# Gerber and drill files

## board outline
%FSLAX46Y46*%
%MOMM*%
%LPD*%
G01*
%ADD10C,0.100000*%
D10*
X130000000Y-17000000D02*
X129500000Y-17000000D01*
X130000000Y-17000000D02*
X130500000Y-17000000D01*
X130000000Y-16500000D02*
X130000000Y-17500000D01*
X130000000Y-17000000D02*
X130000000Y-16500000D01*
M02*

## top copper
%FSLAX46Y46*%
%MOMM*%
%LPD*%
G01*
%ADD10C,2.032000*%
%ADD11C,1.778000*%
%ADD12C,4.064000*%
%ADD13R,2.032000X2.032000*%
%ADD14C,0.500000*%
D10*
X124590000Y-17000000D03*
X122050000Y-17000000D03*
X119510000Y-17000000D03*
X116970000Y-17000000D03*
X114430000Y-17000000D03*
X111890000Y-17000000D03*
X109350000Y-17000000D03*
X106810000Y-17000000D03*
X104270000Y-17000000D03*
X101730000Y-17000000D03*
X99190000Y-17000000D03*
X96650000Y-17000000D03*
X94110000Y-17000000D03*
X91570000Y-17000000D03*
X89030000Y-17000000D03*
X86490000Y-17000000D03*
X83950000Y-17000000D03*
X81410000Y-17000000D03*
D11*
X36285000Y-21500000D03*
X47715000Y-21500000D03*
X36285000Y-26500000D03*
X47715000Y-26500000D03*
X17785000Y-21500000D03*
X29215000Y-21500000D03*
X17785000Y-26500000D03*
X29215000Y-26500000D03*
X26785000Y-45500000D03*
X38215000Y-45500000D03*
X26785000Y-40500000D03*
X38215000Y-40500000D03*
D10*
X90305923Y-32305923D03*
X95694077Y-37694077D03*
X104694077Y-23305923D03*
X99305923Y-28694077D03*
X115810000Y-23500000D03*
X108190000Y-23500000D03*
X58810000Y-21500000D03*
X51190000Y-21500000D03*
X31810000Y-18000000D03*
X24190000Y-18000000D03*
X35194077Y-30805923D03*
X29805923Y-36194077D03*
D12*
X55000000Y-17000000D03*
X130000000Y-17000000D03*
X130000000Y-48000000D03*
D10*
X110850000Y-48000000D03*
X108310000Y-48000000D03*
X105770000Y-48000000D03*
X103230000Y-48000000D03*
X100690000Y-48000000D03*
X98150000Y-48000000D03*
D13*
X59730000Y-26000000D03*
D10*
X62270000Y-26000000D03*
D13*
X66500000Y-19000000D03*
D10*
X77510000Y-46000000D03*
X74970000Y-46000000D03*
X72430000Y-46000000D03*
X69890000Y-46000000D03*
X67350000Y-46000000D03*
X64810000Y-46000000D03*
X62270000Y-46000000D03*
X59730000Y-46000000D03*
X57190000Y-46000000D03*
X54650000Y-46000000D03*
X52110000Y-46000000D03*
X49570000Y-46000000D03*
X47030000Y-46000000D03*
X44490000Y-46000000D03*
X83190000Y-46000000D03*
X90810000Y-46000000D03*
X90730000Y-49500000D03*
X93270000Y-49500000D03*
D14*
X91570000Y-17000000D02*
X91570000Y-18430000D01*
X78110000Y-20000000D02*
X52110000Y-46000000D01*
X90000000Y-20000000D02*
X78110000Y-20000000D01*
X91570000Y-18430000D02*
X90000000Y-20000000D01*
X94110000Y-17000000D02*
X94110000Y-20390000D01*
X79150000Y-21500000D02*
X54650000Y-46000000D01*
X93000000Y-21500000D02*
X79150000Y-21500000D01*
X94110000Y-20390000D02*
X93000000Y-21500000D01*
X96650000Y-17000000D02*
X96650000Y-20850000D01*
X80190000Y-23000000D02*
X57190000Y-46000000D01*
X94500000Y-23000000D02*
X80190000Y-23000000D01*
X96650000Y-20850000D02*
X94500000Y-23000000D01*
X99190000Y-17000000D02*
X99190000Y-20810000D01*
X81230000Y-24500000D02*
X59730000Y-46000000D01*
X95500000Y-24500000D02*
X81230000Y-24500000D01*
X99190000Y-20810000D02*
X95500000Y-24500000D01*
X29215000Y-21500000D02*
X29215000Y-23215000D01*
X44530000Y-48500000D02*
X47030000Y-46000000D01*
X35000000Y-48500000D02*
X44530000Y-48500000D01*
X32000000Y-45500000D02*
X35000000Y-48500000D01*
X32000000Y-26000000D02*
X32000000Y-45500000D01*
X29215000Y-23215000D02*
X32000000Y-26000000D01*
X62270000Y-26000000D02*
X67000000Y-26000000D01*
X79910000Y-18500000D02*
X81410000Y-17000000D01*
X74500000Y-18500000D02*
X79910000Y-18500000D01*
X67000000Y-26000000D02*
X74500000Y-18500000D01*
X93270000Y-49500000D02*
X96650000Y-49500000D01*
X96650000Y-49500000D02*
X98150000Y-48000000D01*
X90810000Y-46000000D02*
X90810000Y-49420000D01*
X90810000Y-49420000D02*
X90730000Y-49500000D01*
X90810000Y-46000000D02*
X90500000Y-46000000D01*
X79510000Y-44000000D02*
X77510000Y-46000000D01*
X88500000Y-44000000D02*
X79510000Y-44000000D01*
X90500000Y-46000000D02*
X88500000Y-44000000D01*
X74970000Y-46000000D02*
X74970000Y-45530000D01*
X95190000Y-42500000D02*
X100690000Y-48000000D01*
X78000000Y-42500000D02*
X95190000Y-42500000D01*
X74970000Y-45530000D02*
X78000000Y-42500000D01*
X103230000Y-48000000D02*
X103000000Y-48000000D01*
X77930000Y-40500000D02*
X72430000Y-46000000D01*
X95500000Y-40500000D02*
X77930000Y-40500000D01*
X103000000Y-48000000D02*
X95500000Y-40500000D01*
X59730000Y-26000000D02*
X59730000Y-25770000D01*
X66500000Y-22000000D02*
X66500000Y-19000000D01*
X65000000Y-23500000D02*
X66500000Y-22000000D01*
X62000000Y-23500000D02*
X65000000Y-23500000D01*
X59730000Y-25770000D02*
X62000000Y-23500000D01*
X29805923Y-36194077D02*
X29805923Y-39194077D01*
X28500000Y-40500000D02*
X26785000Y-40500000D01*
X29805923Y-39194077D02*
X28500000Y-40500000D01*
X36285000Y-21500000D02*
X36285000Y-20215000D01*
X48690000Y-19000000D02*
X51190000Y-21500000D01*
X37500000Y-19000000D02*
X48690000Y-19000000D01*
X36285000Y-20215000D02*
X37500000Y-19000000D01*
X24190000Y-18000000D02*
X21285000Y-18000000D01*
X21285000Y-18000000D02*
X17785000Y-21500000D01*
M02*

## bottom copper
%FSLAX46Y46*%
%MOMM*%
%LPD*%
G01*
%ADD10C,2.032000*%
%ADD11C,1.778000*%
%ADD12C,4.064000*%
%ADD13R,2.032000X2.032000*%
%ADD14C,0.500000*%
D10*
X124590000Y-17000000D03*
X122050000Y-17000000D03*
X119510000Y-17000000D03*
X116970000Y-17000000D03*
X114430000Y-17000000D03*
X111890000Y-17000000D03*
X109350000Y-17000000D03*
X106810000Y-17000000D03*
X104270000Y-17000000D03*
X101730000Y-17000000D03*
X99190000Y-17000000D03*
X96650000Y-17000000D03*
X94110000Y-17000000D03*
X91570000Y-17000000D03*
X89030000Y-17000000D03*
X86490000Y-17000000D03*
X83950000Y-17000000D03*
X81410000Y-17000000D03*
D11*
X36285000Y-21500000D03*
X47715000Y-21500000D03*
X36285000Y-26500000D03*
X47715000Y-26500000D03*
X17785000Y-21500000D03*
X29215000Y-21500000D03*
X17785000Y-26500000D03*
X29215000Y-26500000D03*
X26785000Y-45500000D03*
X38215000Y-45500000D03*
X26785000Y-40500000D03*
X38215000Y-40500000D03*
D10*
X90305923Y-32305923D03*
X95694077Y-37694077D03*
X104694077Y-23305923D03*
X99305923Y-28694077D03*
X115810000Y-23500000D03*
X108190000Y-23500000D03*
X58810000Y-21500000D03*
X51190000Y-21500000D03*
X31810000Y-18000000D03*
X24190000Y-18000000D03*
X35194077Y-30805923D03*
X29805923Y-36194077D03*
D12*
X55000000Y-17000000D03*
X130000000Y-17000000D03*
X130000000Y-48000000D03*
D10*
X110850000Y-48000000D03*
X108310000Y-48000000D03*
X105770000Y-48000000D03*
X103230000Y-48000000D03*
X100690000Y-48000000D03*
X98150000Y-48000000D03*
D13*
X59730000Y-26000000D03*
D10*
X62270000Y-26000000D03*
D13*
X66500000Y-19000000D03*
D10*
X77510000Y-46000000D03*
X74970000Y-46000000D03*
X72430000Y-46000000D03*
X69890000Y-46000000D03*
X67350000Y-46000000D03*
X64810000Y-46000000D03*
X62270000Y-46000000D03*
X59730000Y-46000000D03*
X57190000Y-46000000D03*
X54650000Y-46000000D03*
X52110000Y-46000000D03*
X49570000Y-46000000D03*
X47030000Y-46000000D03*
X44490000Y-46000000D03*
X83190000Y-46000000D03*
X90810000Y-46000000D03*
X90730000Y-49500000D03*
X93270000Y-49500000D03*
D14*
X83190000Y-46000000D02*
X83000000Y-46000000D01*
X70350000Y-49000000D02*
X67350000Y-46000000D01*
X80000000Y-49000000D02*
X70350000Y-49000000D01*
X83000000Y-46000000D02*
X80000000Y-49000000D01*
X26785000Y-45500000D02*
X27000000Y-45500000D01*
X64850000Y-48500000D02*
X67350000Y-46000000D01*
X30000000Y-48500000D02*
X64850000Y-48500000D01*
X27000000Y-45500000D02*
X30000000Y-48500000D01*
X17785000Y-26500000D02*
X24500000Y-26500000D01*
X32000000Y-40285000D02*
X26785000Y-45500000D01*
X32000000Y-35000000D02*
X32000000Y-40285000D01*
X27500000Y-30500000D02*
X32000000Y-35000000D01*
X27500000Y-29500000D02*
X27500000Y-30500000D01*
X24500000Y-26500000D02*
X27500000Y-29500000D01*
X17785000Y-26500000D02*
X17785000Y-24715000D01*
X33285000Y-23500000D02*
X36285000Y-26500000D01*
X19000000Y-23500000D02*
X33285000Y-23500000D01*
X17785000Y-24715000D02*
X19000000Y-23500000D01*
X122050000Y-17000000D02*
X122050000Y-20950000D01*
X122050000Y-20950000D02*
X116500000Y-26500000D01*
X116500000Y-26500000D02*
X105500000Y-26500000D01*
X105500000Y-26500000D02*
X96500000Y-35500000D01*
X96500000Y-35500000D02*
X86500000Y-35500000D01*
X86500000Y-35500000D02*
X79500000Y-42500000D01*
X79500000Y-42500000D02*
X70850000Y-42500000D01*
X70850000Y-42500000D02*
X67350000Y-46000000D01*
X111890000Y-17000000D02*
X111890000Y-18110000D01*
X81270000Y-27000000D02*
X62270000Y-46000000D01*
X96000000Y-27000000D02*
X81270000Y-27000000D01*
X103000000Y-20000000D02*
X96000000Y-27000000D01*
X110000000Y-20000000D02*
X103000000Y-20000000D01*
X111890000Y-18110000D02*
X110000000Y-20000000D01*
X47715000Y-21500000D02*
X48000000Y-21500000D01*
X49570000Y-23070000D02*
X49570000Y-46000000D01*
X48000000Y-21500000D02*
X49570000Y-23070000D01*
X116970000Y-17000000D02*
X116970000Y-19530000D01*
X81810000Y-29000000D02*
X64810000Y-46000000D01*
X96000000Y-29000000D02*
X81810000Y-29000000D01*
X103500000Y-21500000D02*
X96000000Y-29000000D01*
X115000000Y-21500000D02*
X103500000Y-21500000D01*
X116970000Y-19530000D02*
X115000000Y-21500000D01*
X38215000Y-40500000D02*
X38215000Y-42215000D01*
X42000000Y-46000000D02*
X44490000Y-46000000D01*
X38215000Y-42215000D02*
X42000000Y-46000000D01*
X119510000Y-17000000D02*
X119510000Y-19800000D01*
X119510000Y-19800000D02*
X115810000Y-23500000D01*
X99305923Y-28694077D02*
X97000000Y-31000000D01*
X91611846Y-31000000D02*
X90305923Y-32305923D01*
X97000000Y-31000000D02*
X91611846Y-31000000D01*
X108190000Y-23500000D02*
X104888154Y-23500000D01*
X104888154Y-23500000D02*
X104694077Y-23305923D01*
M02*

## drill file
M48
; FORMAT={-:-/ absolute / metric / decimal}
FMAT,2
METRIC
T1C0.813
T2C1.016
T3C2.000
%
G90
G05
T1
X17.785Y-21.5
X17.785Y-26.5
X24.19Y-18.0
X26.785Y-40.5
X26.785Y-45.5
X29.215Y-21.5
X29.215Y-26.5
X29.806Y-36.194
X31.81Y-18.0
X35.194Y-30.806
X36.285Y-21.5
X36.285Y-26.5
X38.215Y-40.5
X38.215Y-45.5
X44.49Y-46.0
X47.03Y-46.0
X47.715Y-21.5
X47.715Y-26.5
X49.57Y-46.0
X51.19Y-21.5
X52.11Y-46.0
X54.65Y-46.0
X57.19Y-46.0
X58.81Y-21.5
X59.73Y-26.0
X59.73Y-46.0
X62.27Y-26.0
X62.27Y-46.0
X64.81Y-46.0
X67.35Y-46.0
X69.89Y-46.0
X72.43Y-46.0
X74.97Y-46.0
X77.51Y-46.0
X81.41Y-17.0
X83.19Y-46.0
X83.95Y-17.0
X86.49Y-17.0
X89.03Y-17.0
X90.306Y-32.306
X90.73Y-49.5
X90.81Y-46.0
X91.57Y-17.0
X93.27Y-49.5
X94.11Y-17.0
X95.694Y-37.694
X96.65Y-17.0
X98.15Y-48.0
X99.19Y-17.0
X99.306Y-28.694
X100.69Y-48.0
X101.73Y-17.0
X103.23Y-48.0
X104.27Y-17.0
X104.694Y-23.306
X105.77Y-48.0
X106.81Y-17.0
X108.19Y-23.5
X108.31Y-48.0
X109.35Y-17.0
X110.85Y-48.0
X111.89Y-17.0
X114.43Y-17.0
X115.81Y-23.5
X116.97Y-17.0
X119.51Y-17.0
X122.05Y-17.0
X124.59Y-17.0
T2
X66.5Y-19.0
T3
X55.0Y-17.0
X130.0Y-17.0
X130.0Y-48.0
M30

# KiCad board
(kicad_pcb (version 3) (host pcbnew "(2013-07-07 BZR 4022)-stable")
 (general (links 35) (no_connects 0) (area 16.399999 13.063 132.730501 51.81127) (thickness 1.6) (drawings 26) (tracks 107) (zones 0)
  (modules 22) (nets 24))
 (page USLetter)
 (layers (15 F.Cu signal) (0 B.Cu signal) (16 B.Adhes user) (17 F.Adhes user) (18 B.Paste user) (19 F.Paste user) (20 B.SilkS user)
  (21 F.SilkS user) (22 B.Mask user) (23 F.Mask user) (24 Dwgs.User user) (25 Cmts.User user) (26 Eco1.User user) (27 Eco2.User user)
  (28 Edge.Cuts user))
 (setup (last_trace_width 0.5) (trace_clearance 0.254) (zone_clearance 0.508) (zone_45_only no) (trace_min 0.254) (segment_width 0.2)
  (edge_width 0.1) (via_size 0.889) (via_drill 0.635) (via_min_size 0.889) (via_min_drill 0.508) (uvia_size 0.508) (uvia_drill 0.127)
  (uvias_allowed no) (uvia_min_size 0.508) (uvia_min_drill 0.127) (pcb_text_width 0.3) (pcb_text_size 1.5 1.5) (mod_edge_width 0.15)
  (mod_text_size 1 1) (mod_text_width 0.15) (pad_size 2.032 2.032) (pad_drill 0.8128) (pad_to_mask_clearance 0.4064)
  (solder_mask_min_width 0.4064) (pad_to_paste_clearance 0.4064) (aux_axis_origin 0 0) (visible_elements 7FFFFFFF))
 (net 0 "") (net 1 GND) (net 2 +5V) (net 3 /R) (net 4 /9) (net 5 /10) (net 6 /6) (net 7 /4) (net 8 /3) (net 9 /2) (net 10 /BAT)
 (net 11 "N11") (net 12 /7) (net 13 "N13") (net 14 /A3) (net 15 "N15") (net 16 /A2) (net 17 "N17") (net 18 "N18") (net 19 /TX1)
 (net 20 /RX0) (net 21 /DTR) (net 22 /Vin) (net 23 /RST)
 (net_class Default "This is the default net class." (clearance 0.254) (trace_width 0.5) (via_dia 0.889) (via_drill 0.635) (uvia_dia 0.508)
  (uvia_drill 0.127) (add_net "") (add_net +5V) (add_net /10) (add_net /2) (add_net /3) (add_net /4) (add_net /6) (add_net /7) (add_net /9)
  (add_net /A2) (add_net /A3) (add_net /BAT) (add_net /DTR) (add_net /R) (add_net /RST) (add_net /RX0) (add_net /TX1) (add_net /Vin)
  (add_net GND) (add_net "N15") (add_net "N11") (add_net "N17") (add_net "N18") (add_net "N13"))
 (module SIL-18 (layer F.Cu) (at 103 17 180) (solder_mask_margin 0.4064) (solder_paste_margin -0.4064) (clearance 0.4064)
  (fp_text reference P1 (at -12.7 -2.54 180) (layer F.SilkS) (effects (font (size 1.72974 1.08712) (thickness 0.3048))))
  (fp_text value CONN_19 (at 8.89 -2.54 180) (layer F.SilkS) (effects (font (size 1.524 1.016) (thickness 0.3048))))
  (pad 1 thru_hole circle (at -21.59 0 180) (size 2.032 2.032) (drill 0.8128) (layers *.Cu *.Mask F.SilkS) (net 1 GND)
   (solder_mask_margin 0.4064) (solder_paste_margin -0.4064) (clearance 0.4064) (zone_connect 1) (thermal_width 0.508) (thermal_gap 0.508))
  (pad 2 thru_hole circle (at -19.05 0 180) (size 2.032 2.032) (drill 0.8128) (layers *.Cu *.Mask F.SilkS) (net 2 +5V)
   (solder_mask_margin 0.4064) (solder_paste_margin -0.4064) (clearance 0.4064) (zone_connect 1) (thermal_width 0.508) (thermal_gap 0.508))
  (pad 3 thru_hole circle (at -16.51 0 180) (size 2.032 2.032) (drill 0.8128) (layers *.Cu *.Mask F.SilkS) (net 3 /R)
   (solder_mask_margin 0.4064) (solder_paste_margin -0.4064) (clearance 0.4064) (zone_connect 1) (thermal_width 0.508) (thermal_gap 0.508))
  (pad 4 thru_hole circle (at -13.97 0 180) (size 2.032 2.032) (drill 0.8128) (layers *.Cu *.Mask F.SilkS) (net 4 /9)
   (solder_mask_margin 0.4064) (solder_paste_margin -0.4064) (clearance 0.4064) (zone_connect 1) (thermal_width 0.508) (thermal_gap 0.508))
  (pad 5 thru_hole circle (at -11.43 0 180) (size 2.032 2.032) (drill 0.8128) (layers *.Cu *.Mask F.SilkS) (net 1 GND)
   (solder_mask_margin 0.4064) (solder_paste_margin -0.4064) (clearance 0.4064) (zone_connect 1) (thermal_width 0.508) (thermal_gap 0.508))
  (pad 6 thru_hole circle (at -8.89 0 180) (size 2.032 2.032) (drill 0.8128) (layers *.Cu *.Mask F.SilkS) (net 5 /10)
   (solder_mask_margin 0.4064) (solder_paste_margin -0.4064) (clearance 0.4064) (zone_connect 1) (thermal_width 0.508) (thermal_gap 0.508))
  (pad 7 thru_hole circle (at -6.35 0 180) (size 2.032 2.032) (drill 0.8128) (layers *.Cu *.Mask F.SilkS) (solder_mask_margin 0.4064)
   (solder_paste_margin -0.4064) (clearance 0.4064) (zone_connect 1) (thermal_width 0.508) (thermal_gap 0.508))
  (pad 8 thru_hole circle (at -3.81 0 180) (size 2.032 2.032) (drill 0.8128) (layers *.Cu *.Mask F.SilkS) (solder_mask_margin 0.4064)
   (solder_paste_margin -0.4064) (clearance 0.4064) (zone_connect 1) (thermal_width 0.508) (thermal_gap 0.508))
  (pad 9 thru_hole circle (at -1.27 0 180) (size 2.032 2.032) (drill 0.8128) (layers *.Cu *.Mask F.SilkS) (solder_mask_margin 0.4064)
   (solder_paste_margin -0.4064) (clearance 0.4064) (zone_connect 1) (thermal_width 0.508) (thermal_gap 0.508))
  (pad 10 thru_hole circle (at 1.27 0 180) (size 2.032 2.032) (drill 0.8128) (layers *.Cu *.Mask F.SilkS) (solder_mask_margin 0.4064)
   (solder_paste_margin -0.4064) (clearance 0.4064) (zone_connect 1) (thermal_width 0.508) (thermal_gap 0.508))
  (pad 11 thru_hole circle (at 3.81 0 180) (size 2.032 2.032) (drill 0.8128) (layers *.Cu *.Mask F.SilkS) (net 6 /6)
   (solder_mask_margin 0.4064) (solder_paste_margin -0.4064) (clearance 0.4064) (zone_connect 1) (thermal_width 0.508) (thermal_gap 0.508))
  (pad 12 thru_hole circle (at 6.35 0 180) (size 2.032 2.032) (drill 0.8128) (layers *.Cu *.Mask F.SilkS) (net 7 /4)
   (solder_mask_margin 0.4064) (solder_paste_margin -0.4064) (clearance 0.4064) (zone_connect 1) (thermal_width 0.508) (thermal_gap 0.508))
  (pad 13 thru_hole circle (at 8.89 0 180) (size 2.032 2.032) (drill 0.8128) (layers *.Cu *.Mask F.SilkS) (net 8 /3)
   (solder_mask_margin 0.4064) (solder_paste_margin -0.4064) (clearance 0.4064) (zone_connect 1) (thermal_width 0.508) (thermal_gap 0.508))
  (pad 14 thru_hole circle (at 11.43 0 180) (size 2.032 2.032) (drill 0.8128) (layers *.Cu *.Mask F.SilkS) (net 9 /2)
   (solder_mask_margin 0.4064) (solder_paste_margin -0.4064) (clearance 0.4064) (thermal_width 0.508) (thermal_gap 0.508))
  (pad 15 thru_hole circle (at 13.97 0 180) (size 2.032 2.032) (drill 0.8128) (layers *.Cu *.Mask F.SilkS) (solder_mask_margin 0.4064)
   (solder_paste_margin -0.4064) (clearance 0.4064) (zone_connect 1) (thermal_width 0.508) (thermal_gap 0.508))
  (pad 16 thru_hole circle (at 16.51 0 180) (size 2.032 2.032) (drill 0.8128) (layers *.Cu *.Mask F.SilkS) (solder_mask_margin 0.4064)
   (solder_paste_margin -0.4064) (clearance 0.4064) (zone_connect 1) (thermal_width 0.508) (thermal_gap 0.508))
  (pad 17 thru_hole circle (at 19.05 0 180) (size 2.032 2.032) (drill 0.8128) (layers *.Cu *.Mask F.SilkS) (solder_mask_margin 0.4064)
   (solder_paste_margin -0.4064) (clearance 0.4064) (zone_connect 1) (thermal_width 0.508) (thermal_gap 0.508))
  (pad 18 thru_hole circle (at 21.59 0 180) (size 2.032 2.032) (drill 0.8128) (layers *.Cu *.Mask F.SilkS) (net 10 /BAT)
   (solder_mask_margin 0.4064) (solder_paste_margin -0.4064) (clearance 0.4064) (zone_connect 1) (thermal_width 0.508) (thermal_gap 0.508)))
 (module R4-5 (layer F.Cu) (at 42 21.5)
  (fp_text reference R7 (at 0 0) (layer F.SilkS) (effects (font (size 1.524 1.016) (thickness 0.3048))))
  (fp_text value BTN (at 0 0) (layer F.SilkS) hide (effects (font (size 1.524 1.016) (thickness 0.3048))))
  (pad 1 thru_hole circle (at -5.715 0) (size 1.778 1.778) (drill 0.8128) (layers *.Cu *.Mask F.SilkS) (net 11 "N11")
   (solder_mask_margin 0.4064) (solder_paste_margin -0.4064) (clearance 0.4064) (zone_connect 1) (thermal_width 0.508) (thermal_gap 0.508))
  (pad 2 thru_hole circle (at 5.715 0) (size 1.778 1.778) (drill 0.8128) (layers *.Cu *.Mask F.SilkS) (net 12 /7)
   (solder_mask_margin 0.4064) (solder_paste_margin -0.4064) (clearance 0.4064) (zone_connect 1) (thermal_width 0.508) (thermal_gap 0.508)))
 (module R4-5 (layer F.Cu) (at 42 26.5)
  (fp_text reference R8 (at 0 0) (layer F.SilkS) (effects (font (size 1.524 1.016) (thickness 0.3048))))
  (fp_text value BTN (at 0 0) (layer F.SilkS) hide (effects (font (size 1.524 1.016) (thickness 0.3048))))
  (pad 1 thru_hole circle (at -5.715 0) (size 1.778 1.778) (drill 0.8128) (layers *.Cu *.Mask F.SilkS) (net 2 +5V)
   (solder_mask_margin 0.4064) (solder_paste_margin -0.4064) (clearance 0.4064) (thermal_width 0.508) (thermal_gap 0.508))
  (pad 2 thru_hole circle (at 5.715 0) (size 1.778 1.778) (drill 0.8128) (layers *.Cu *.Mask F.SilkS) (solder_mask_margin 0.4064)
   (solder_paste_margin -0.4064) (clearance 0.4064) (thermal_width 0.508) (thermal_gap 0.508)))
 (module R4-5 (layer F.Cu) (at 23.5 21.5)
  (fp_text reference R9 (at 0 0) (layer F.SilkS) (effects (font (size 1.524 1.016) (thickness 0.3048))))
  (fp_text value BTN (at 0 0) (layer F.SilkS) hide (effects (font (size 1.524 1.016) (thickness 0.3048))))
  (pad 1 thru_hole circle (at -5.715 0) (size 1.778 1.778) (drill 0.8128) (layers *.Cu *.Mask F.SilkS) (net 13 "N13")
   (solder_mask_margin 0.4064) (solder_paste_margin -0.4064) (clearance 0.4064) (zone_connect 1) (thermal_width 0.4064) (thermal_gap 0.4064))
  (pad 2 thru_hole circle (at 5.715 0) (size 1.778 1.778) (drill 0.8128) (layers *.Cu *.Mask F.SilkS) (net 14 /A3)
   (solder_mask_margin 0.4064) (solder_paste_margin -0.4064) (clearance 0.4064) (zone_connect 1) (thermal_width 0.508) (thermal_gap 0.508)))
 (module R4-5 (layer F.Cu) (at 23.5 26.5)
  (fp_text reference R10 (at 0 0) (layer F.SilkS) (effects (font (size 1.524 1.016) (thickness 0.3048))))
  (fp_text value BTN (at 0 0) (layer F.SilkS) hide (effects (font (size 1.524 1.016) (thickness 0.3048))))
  (pad 1 thru_hole circle (at -5.715 0) (size 1.778 1.778) (drill 0.8128) (layers *.Cu *.Mask F.SilkS) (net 2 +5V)
   (solder_mask_margin 0.4064) (solder_paste_margin -0.4064) (clearance 0.4064) (zone_connect 1) (thermal_width 0.508) (thermal_gap 0.508))
  (pad 2 thru_hole circle (at 5.715 0) (size 1.778 1.778) (drill 0.8128) (layers *.Cu *.Mask F.SilkS) (solder_mask_margin 0.4064)
   (solder_paste_margin -0.4064) (clearance 0.4064) (zone_connect 1) (thermal_width 0.508) (thermal_gap 0.508)))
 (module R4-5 (layer F.Cu) (at 32.5 45.5)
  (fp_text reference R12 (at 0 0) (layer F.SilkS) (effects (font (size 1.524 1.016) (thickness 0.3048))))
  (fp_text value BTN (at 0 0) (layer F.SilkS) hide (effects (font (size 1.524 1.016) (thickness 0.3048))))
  (pad 1 thru_hole circle (at -5.715 0) (size 1.778 1.778) (drill 0.8128) (layers *.Cu *.Mask F.SilkS) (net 2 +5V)
   (solder_mask_margin 0.4064) (solder_paste_margin -0.4064) (clearance 0.4064) (zone_connect 1) (thermal_width 0.508) (thermal_gap 0.508))
  (pad 2 thru_hole circle (at 5.715 0) (size 1.778 1.778) (drill 0.8128) (layers *.Cu *.Mask F.SilkS) (solder_mask_margin 0.4064)
   (solder_paste_margin -0.4064) (clearance 0.4064) (zone_connect 1) (thermal_width 0.508) (thermal_gap 0.508)))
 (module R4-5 (layer F.Cu) (at 32.5 40.5)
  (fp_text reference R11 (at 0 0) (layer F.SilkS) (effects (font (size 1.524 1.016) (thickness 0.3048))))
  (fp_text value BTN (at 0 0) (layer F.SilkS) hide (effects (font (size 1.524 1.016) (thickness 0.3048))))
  (pad 1 thru_hole circle (at -5.715 0) (size 1.778 1.778) (drill 0.8128) (layers *.Cu *.Mask F.SilkS) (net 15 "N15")
   (solder_mask_margin 0.4064) (solder_paste_margin -0.4064) (clearance 0.4064) (zone_connect 1) (thermal_width 0.508) (thermal_gap 0.508))
  (pad 2 thru_hole circle (at 5.715 0) (size 1.778 1.778) (drill 0.8128) (layers *.Cu *.Mask F.SilkS) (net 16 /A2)
   (solder_mask_margin 0.4064) (solder_paste_margin -0.4064) (clearance 0.4064) (zone_connect 1) (thermal_width 0.508) (thermal_gap 0.508)))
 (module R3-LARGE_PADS (layer F.Cu) (at 93 35 315) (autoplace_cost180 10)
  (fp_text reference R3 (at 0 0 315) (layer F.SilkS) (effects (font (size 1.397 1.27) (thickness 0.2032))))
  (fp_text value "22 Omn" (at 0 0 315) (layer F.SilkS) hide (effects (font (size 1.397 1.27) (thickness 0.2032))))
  (pad 1 thru_hole circle (at -3.81 0 315) (size 2.032 2.032) (drill 0.8128) (layers *.Cu *.Mask F.SilkS) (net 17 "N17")
   (solder_mask_margin 0.4064) (solder_paste_margin -0.4064) (clearance 0.4064) (zone_connect 1) (thermal_width 0.508) (thermal_gap 0.508))
  (pad 2 thru_hole circle (at 3.81 0 315) (size 2.032 2.032) (drill 0.8128) (layers *.Cu *.Mask F.SilkS) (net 1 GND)
   (solder_mask_margin 0.4064) (solder_paste_margin -0.4064) (clearance 0.4064) (zone_connect 1) (thermal_width 0.508) (thermal_gap 0.508)))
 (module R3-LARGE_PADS (layer F.Cu) (at 102 26 225) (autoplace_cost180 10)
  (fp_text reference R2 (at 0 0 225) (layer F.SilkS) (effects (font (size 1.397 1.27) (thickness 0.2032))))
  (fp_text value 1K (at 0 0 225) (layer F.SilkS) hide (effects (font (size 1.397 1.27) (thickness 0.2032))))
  (pad 1 thru_hole circle (at -3.81 0 225) (size 2.032 2.032) (drill 0.8128) (layers *.Cu *.Mask F.SilkS) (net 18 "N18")
   (solder_mask_margin 0.4064) (solder_paste_margin -0.4064) (clearance 0.4064) (zone_connect 1) (thermal_width 0.508) (thermal_gap 0.508))
  (pad 2 thru_hole circle (at 3.81 0 225) (size 2.032 2.032) (drill 0.8128) (layers *.Cu *.Mask F.SilkS) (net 17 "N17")
   (solder_mask_margin 0.4064) (solder_paste_margin -0.4064) (clearance 0.4064) (zone_connect 1) (thermal_width 0.508) (thermal_gap 0.508)))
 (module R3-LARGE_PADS (layer F.Cu) (at 112 23.5 180) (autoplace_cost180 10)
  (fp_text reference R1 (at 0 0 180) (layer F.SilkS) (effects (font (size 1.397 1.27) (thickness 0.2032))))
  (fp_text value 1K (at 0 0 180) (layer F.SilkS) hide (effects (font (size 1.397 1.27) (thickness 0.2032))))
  (pad 1 thru_hole circle (at -3.81 0 180) (size 2.032 2.032) (drill 0.8128) (layers *.Cu *.Mask F.SilkS) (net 3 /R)
   (solder_mask_margin 0.4064) (solder_paste_margin -0.4064) (clearance 0.4064) (zone_connect 1) (thermal_width 0.508) (thermal_gap 0.508))
  (pad 2 thru_hole circle (at 3.81 0 180) (size 2.032 2.032) (drill 0.8128) (layers *.Cu *.Mask F.SilkS) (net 18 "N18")
   (solder_mask_margin 0.4064) (solder_paste_margin -0.4064) (clearance 0.4064) (zone_connect 1) (thermal_width 0.508) (thermal_gap 0.508)))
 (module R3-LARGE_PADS (layer F.Cu) (at 55 21.5 180) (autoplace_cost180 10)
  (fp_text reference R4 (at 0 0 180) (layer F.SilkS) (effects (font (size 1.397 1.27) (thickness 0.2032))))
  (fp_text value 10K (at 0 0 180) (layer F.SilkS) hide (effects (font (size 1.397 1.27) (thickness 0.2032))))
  (pad 1 thru_hole circle (at -3.81 0 180) (size 2.032 2.032) (drill 0.8128) (layers *.Cu *.Mask F.SilkS) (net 1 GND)
   (solder_mask_margin 0.4064) (solder_paste_margin -0.4064) (clearance 0.4064) (zone_connect 1) (thermal_width 0.508) (thermal_gap 0.508))
  (pad 2 thru_hole circle (at 3.81 0 180) (size 2.032 2.032) (drill 0.8128) (layers *.Cu *.Mask F.SilkS) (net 11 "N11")
   (solder_mask_margin 0.4064) (solder_paste_margin -0.4064) (clearance 0.4064) (zone_connect 1) (thermal_width 0.508) (thermal_gap 0.508)))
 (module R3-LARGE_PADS (layer F.Cu) (at 28 18 180) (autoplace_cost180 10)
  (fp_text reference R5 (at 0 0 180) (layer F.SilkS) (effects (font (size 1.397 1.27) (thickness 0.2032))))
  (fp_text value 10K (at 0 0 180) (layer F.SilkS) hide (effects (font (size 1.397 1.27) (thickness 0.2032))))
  (pad 1 thru_hole circle (at -3.81 0 180) (size 2.032 2.032) (drill 0.8128) (layers *.Cu *.Mask F.SilkS) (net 1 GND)
   (solder_mask_margin 0.4064) (solder_paste_margin -0.4064) (clearance 0.4064) (zone_connect 1) (thermal_width 0.508) (thermal_gap 0.508))
  (pad 2 thru_hole circle (at 3.81 0 180) (size 2.032 2.032) (drill 0.8128) (layers *.Cu *.Mask F.SilkS) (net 13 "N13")
   (solder_mask_margin 0.4064) (solder_paste_margin -0.4064) (clearance 0.4064) (thermal_width 0.508) (thermal_gap 0.508)))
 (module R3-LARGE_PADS (layer F.Cu) (at 32.5 33.5 225) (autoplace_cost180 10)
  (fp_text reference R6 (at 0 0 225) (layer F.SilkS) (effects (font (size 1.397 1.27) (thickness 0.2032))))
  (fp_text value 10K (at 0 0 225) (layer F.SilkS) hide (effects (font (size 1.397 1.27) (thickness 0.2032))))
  (pad 1 thru_hole circle (at -3.81 0 225) (size 2.032 2.032) (drill 0.8128) (layers *.Cu *.Mask F.SilkS) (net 1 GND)
   (solder_mask_margin 0.4064) (solder_paste_margin -0.4064) (clearance 0.4064) (zone_connect 1) (thermal_width 0.508) (thermal_gap 0.508))
  (pad 2 thru_hole circle (at 3.81 0 225) (size 2.032 2.032) (drill 0.8128) (layers *.Cu *.Mask F.SilkS) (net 15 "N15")
   (solder_mask_margin 0.4064) (solder_paste_margin -0.4064) (clearance 0.4064) (zone_connect 1) (thermal_width 0.508) (thermal_gap 0.508)))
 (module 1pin (layer F.Cu) (at 55 17)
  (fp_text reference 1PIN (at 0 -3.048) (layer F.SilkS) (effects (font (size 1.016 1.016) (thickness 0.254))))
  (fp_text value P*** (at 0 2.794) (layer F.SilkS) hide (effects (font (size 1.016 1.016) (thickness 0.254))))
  (pad 1 thru_hole circle (at 0 0) (size 4.064 4.064) (drill 2) (layers *.Cu *.Mask F.SilkS)))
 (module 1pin (layer F.Cu) (at 130 17)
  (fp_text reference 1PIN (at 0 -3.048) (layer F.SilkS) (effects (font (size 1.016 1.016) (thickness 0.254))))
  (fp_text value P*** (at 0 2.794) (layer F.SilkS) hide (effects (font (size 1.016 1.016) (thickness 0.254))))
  (pad 1 thru_hole circle (at 0 0) (size 4.064 4.064) (drill 2) (layers *.Cu *.Mask F.SilkS)))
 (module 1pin (layer F.Cu) (at 130 48)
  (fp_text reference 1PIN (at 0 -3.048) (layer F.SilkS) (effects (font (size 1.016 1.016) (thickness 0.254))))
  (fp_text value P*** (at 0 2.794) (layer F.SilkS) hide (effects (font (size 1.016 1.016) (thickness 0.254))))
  (pad 1 thru_hole circle (at 0 0) (size 4.064 4.064) (drill 2) (layers *.Cu *.Mask F.SilkS)))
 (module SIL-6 (layer F.Cu) (at 104.5 48 180)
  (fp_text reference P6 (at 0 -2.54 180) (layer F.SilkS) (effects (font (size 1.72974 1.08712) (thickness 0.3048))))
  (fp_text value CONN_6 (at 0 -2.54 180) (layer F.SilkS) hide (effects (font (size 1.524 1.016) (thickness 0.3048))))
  (pad 1 thru_hole circle (at -6.35 0 180) (size 2.032 2.032) (drill 0.8128) (layers *.Cu *.Mask F.SilkS) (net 1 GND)
   (solder_mask_margin 0.4064) (solder_paste_margin -0.4064) (clearance 0.4064) (zone_connect 1) (thermal_width 0.508) (thermal_gap 0.508))
  (pad 2 thru_hole circle (at -3.81 0 180) (size 2.032 2.032) (drill 0.8128) (layers *.Cu *.Mask F.SilkS) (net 1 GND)
   (solder_mask_margin 0.4064) (solder_paste_margin -0.4064) (clearance 0.4064) (zone_connect 1) (thermal_width 0.508) (thermal_gap 0.508))
  (pad 3 thru_hole circle (at -1.27 0 180) (size 2.032 2.032) (drill 0.8128) (layers *.Cu *.Mask F.SilkS) (solder_mask_margin 0.4064)
   (solder_paste_margin -0.4064) (clearance 0.4064) (zone_connect 1) (thermal_width 0.508) (thermal_gap 0.508))
  (pad 4 thru_hole circle (at 1.27 0 180) (size 2.032 2.032) (drill 0.8128) (layers *.Cu *.Mask F.SilkS) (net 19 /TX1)
   (solder_mask_margin 0.4064) (solder_paste_margin -0.4064) (clearance 0.4064) (zone_connect 1) (thermal_width 0.508) (thermal_gap 0.508))
  (pad 5 thru_hole circle (at 3.81 0 180) (size 2.032 2.032) (drill 0.8128) (layers *.Cu *.Mask F.SilkS) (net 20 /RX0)
   (solder_mask_margin 0.4064) (solder_paste_margin -0.4064) (clearance 0.4064) (zone_connect 1) (thermal_width 0.508) (thermal_gap 0.508))
  (pad 6 thru_hole circle (at 6.35 0 180) (size 2.032 2.032) (drill 0.8128) (layers *.Cu *.Mask F.SilkS) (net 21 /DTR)
   (solder_mask_margin 0.4064) (solder_paste_margin -0.4064) (clearance 0.4064) (zone_connect 1) (thermal_width 0.508) (thermal_gap 0.508)))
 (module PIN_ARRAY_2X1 (layer F.Cu) (at 61 26)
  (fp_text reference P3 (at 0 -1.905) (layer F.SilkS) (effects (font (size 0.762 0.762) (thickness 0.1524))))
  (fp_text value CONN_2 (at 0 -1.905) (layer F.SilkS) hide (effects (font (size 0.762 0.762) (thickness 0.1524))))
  (pad 1 thru_hole rect (at -1.27 0) (size 2.032 2.032) (drill 0.8128) (layers *.Cu *.Mask F.SilkS) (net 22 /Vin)
   (solder_mask_margin 0.4064) (solder_paste_margin -0.4064) (clearance 0.4064) (thermal_width 0.508) (thermal_gap 0.508))
  (pad 2 thru_hole circle (at 1.27 0) (size 2.032 2.032) (drill 0.8128) (layers *.Cu *.Mask F.SilkS) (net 10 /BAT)
   (solder_mask_margin 0.4064) (solder_paste_margin -0.4064) (clearance 0.4064) (thermal_width 0.508) (thermal_gap 0.508)))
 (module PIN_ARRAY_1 (layer F.Cu) (at 66.5 19)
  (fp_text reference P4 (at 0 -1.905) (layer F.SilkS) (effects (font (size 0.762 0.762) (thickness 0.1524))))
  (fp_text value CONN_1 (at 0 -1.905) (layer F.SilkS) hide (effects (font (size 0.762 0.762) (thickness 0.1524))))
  (pad 1 thru_hole rect (at 0 0) (size 2.032 2.032) (drill 1.016) (layers *.Cu *.Mask F.SilkS) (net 22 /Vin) (solder_mask_margin 0.4064)
   (solder_paste_margin -0.4064) (clearance 0.4064) (thermal_width 0.508) (thermal_gap 0.508)))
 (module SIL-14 (layer F.Cu) (at 61 46 180)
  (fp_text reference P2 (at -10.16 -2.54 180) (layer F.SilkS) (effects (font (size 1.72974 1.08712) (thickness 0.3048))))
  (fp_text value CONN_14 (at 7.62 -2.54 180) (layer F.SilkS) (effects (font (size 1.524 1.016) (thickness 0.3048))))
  (pad 1 thru_hole circle (at -16.51 0 180) (size 2.032 2.032) (drill 0.8128) (layers *.Cu *.Mask F.SilkS) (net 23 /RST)
   (solder_mask_margin 0.4064) (solder_paste_margin -0.4064) (clearance 0.4064) (zone_connect 1) (thermal_width 0.508) (thermal_gap 0.508))
  (pad 2 thru_hole circle (at -13.97 0 180) (size 2.032 2.032) (drill 0.8128) (layers *.Cu *.Mask F.SilkS) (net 20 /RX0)
   (solder_mask_margin 0.4064) (solder_paste_margin -0.4064) (clearance 0.4064) (zone_connect 1) (thermal_width 0.508) (thermal_gap 0.508))
  (pad 3 thru_hole circle (at -11.43 0 180) (size 2.032 2.032) (drill 0.8128) (layers *.Cu *.Mask F.SilkS) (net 19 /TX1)
   (solder_mask_margin 0.4064) (solder_paste_margin -0.4064) (clearance 0.4064) (zone_connect 1) (thermal_width 0.508) (thermal_gap 0.508))
  (pad 4 thru_hole circle (at -8.89 0 180) (size 2.032 2.032) (drill 0.8128) (layers *.Cu *.Mask F.SilkS) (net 1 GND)
   (solder_mask_margin 0.4064) (solder_paste_margin -0.4064) (clearance 0.4064) (zone_connect 1) (thermal_width 0.508) (thermal_gap 0.508))
  (pad 5 thru_hole circle (at -6.35 0 180) (size 2.032 2.032) (drill 0.8128) (layers *.Cu *.Mask F.SilkS) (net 2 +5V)
   (solder_mask_margin 0.4064) (solder_paste_margin -0.4064) (clearance 0.4064) (zone_connect 1) (thermal_width 0.508) (thermal_gap 0.508))
  (pad 6 thru_hole circle (at -3.81 0 180) (size 2.032 2.032) (drill 0.8128) (layers *.Cu *.Mask F.SilkS) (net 4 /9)
   (solder_mask_margin 0.4064) (solder_paste_margin -0.4064) (clearance 0.4064) (zone_connect 1) (thermal_width 0.508) (thermal_gap 0.508))
  (pad 7 thru_hole circle (at -1.27 0 180) (size 2.032 2.032) (drill 0.8128) (layers *.Cu *.Mask F.SilkS) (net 5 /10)
   (solder_mask_margin 0.4064) (solder_paste_margin -0.4064) (clearance 0.4064) (zone_connect 1) (thermal_width 0.508) (thermal_gap 0.508))
  (pad 8 thru_hole circle (at 1.27 0 180) (size 2.032 2.032) (drill 0.8128) (layers *.Cu *.Mask F.SilkS) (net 6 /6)
   (solder_mask_margin 0.4064) (solder_paste_margin -0.4064) (clearance 0.4064) (zone_connect 1) (thermal_width 0.508) (thermal_gap 0.508))
  (pad 9 thru_hole circle (at 3.81 0 180) (size 2.032 2.032) (drill 0.8128) (layers *.Cu *.Mask F.SilkS) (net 7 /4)
   (solder_mask_margin 0.4064) (solder_paste_margin -0.4064) (clearance 0.4064) (zone_connect 1) (thermal_width 0.508) (thermal_gap 0.508))
  (pad 10 thru_hole circle (at 6.35 0 180) (size 2.032 2.032) (drill 0.8128) (layers *.Cu *.Mask F.SilkS) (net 8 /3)
   (solder_mask_margin 0.4064) (solder_paste_margin -0.4064) (clearance 0.4064) (zone_connect 1) (thermal_width 0.508) (thermal_gap 0.508))
  (pad 11 thru_hole circle (at 8.89 0 180) (size 2.032 2.032) (drill 0.8128) (layers *.Cu *.Mask F.SilkS) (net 9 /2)
   (solder_mask_margin 0.4064) (solder_paste_margin -0.4064) (clearance 0.4064) (zone_connect 1) (thermal_width 0.508) (thermal_gap 0.508))
  (pad 12 thru_hole circle (at 11.43 0 180) (size 2.032 2.032) (drill 0.8128) (layers *.Cu *.Mask F.SilkS) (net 12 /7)
   (solder_mask_margin 0.4064) (solder_paste_margin -0.4064) (clearance 0.4064) (zone_connect 1) (thermal_width 0.508) (thermal_gap 0.508))
  (pad 13 thru_hole circle (at 13.97 0 180) (size 2.032 2.032) (drill 0.8128) (layers *.Cu *.Mask F.SilkS) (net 14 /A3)
   (solder_mask_margin 0.4064) (solder_paste_margin -0.4064) (clearance 0.4064) (zone_connect 1) (thermal_width 0.508) (thermal_gap 0.508))
  (pad 14 thru_hole circle (at 16.51 0 180) (size 2.032 2.032) (drill 0.8128) (layers *.Cu *.Mask F.SilkS) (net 16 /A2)
   (solder_mask_margin 0.4064) (solder_paste_margin -0.4064) (clearance 0.4064) (zone_connect 1) (thermal_width 0.508) (thermal_gap 0.508)))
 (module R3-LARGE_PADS (layer F.Cu) (at 87 46) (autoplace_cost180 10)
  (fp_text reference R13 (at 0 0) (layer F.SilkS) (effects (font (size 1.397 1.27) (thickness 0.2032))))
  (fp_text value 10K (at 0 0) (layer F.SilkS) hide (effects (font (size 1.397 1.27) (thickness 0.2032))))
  (pad 1 thru_hole circle (at -3.81 0) (size 2.032 2.032) (drill 0.8128) (layers *.Cu *.Mask F.SilkS) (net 2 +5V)
   (solder_mask_margin 0.4064) (solder_paste_margin -0.4064) (clearance 0.4064) (zone_connect 1) (thermal_width 0.508) (thermal_gap 0.508))
  (pad 2 thru_hole circle (at 3.81 0) (size 2.032 2.032) (drill 0.8128) (layers *.Cu *.Mask F.SilkS) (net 23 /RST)
   (solder_mask_margin 0.4064) (solder_paste_margin -0.4064) (clearance 0.4064) (zone_connect 1) (thermal_width 0.508) (thermal_gap 0.508)))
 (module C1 (layer F.Cu) (at 92 49.5)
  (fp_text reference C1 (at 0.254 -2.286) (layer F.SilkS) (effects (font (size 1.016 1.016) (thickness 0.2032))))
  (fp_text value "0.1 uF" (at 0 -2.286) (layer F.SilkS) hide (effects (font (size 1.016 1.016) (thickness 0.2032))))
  (pad 1 thru_hole circle (at -1.27 0) (size 2.032 2.032) (drill 0.8128) (layers *.Cu *.Mask F.SilkS) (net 23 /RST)
   (solder_mask_margin 0.4064) (solder_paste_margin -0.4064) (clearance 0.4064) (zone_connect 1) (thermal_width 0.508) (thermal_gap 0.508))
  (pad 2 thru_hole circle (at 1.27 0) (size 2.032 2.032) (drill 0.8128) (layers *.Cu *.Mask F.SilkS) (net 21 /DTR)
   (solder_mask_margin 0.4064) (solder_paste_margin -0.4064) (clearance 0.4064) (zone_connect 1) (thermal_width 0.508) (thermal_gap 0.508)))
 (gr_line (start 130 17) (end 129.5 17) (angle 90) (layer Edge.Cuts) (width 0.1))
 (gr_line (start 130 17) (end 130.5 17) (angle 90) (layer Edge.Cuts) (width 0.1))
 (gr_line (start 130 16.5) (end 130 17.5) (angle 90) (layer Edge.Cuts) (width 0.1))
 (gr_line (start 130 17) (end 130 16.5) (angle 90) (layer Edge.Cuts) (width 0.1))
 (segment (start 83.19 46) (end 83 46) (width 0.5) (layer B.Cu) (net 2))
 (segment (start 70.35 49) (end 67.35 46) (width 0.5) (layer B.Cu) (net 2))
 (segment (start 80 49) (end 70.35 49) (width 0.5) (layer B.Cu) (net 2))
 (segment (start 83 46) (end 80 49) (width 0.5) (layer B.Cu) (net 2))
 (segment (start 26.785 45.5) (end 27 45.5) (width 0.5) (layer B.Cu) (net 2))
 (segment (start 64.85 48.5) (end 67.35 46) (width 0.5) (layer B.Cu) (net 2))
 (segment (start 30 48.5) (end 64.85 48.5) (width 0.5) (layer B.Cu) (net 2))
 (segment (start 27 45.5) (end 30 48.5) (width 0.5) (layer B.Cu) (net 2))
 (segment (start 17.785 26.5) (end 24.5 26.5) (width 0.5) (layer B.Cu) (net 2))
 (segment (start 32 40.285) (end 26.785 45.5) (width 0.5) (layer B.Cu) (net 2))
 (segment (start 32 35) (end 32 40.285) (width 0.5) (layer B.Cu) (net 2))
 (segment (start 27.5 30.5) (end 32 35) (width 0.5) (layer B.Cu) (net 2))
 (segment (start 27.5 29.5) (end 27.5 30.5) (width 0.5) (layer B.Cu) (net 2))
 (segment (start 24.5 26.5) (end 27.5 29.5) (width 0.5) (layer B.Cu) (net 2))
 (segment (start 17.785 26.5) (end 17.785 24.715) (width 0.5) (layer B.Cu) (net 2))
 (segment (start 33.285 23.5) (end 36.285 26.5) (width 0.5) (layer B.Cu) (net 2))
 (segment (start 19 23.5) (end 33.285 23.5) (width 0.5) (layer B.Cu) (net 2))
 (segment (start 17.785 24.715) (end 19 23.5) (width 0.5) (layer B.Cu) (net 2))
 (segment (start 122.05 17) (end 122.05 20.95) (width 0.5) (layer B.Cu) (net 2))
 (segment (start 122.05 20.95) (end 116.5 26.5) (width 0.5) (layer B.Cu) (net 2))
 (segment (start 116.5 26.5) (end 105.5 26.5) (width 0.5) (layer B.Cu) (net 2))
 (segment (start 105.5 26.5) (end 96.5 35.5) (width 0.5) (layer B.Cu) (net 2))
 (segment (start 96.5 35.5) (end 86.5 35.5) (width 0.5) (layer B.Cu) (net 2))
 (segment (start 86.5 35.5) (end 79.5 42.5) (width 0.5) (layer B.Cu) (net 2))
 (segment (start 79.5 42.5) (end 70.85 42.5) (width 0.5) (layer B.Cu) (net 2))
 (segment (start 70.85 42.5) (end 67.35 46) (width 0.5) (layer B.Cu) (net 2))
 (segment (start 111.89 17) (end 111.89 18.11) (width 0.5) (layer B.Cu) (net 5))
 (segment (start 81.27 27) (end 62.27 46) (width 0.5) (layer B.Cu) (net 5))
 (segment (start 96 27) (end 81.27 27) (width 0.5) (layer B.Cu) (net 5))
 (segment (start 103 20) (end 96 27) (width 0.5) (layer B.Cu) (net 5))
 (segment (start 110 20) (end 103 20) (width 0.5) (layer B.Cu) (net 5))
 (segment (start 111.89 18.11) (end 110 20) (width 0.5) (layer B.Cu) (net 5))
 (segment (start 91.57 17) (end 91.57 18.43) (width 0.5) (layer F.Cu) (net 9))
 (segment (start 78.11 20) (end 52.11 46) (width 0.5) (layer F.Cu) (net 9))
 (segment (start 90 20) (end 78.11 20) (width 0.5) (layer F.Cu) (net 9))
 (segment (start 91.57 18.43) (end 90 20) (width 0.5) (layer F.Cu) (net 9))
 (segment (start 94.11 17) (end 94.11 20.39) (width 0.5) (layer F.Cu) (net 8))
 (segment (start 79.15 21.5) (end 54.65 46) (width 0.5) (layer F.Cu) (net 8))
 (segment (start 93 21.5) (end 79.15 21.5) (width 0.5) (layer F.Cu) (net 8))
 (segment (start 94.11 20.39) (end 93 21.5) (width 0.5) (layer F.Cu) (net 8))
 (segment (start 96.65 17) (end 96.65 20.85) (width 0.5) (layer F.Cu) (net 7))
 (segment (start 80.19 23) (end 57.19 46) (width 0.5) (layer F.Cu) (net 7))
 (segment (start 94.5 23) (end 80.19 23) (width 0.5) (layer F.Cu) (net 7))
 (segment (start 96.65 20.85) (end 94.5 23) (width 0.5) (layer F.Cu) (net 7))
 (segment (start 99.19 17) (end 99.19 20.81) (width 0.5) (layer F.Cu) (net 6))
 (segment (start 81.23 24.5) (end 59.73 46) (width 0.5) (layer F.Cu) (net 6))
 (segment (start 95.5 24.5) (end 81.23 24.5) (width 0.5) (layer F.Cu) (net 6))
 (segment (start 99.19 20.81) (end 95.5 24.5) (width 0.5) (layer F.Cu) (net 6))
 (segment (start 47.715 21.5) (end 48 21.5) (width 0.5) (layer B.Cu) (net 12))
 (segment (start 49.57 23.07) (end 49.57 46) (width 0.5) (layer B.Cu) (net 12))
 (segment (start 48 21.5) (end 49.57 23.07) (width 0.5) (layer B.Cu) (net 12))
 (segment (start 116.97 17) (end 116.97 19.53) (width 0.5) (layer B.Cu) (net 4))
 (segment (start 81.81 29) (end 64.81 46) (width 0.5) (layer B.Cu) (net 4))
 (segment (start 96 29) (end 81.81 29) (width 0.5) (layer B.Cu) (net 4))
 (segment (start 103.5 21.5) (end 96 29) (width 0.5) (layer B.Cu) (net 4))
 (segment (start 115 21.5) (end 103.5 21.5) (width 0.5) (layer B.Cu) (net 4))
 (segment (start 116.97 19.53) (end 115 21.5) (width 0.5) (layer B.Cu) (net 4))
 (segment (start 38.215 40.5) (end 38.215 42.215) (width 0.5) (layer B.Cu) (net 16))
 (segment (start 42 46) (end 44.49 46) (width 0.5) (layer B.Cu) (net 16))
 (segment (start 38.215 42.215) (end 42 46) (width 0.5) (layer B.Cu) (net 16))
 (segment (start 29.215 21.5) (end 29.215 23.215) (width 0.5) (layer F.Cu) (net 14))
 (segment (start 44.53 48.5) (end 47.03 46) (width 0.5) (layer F.Cu) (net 14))
 (segment (start 35 48.5) (end 44.53 48.5) (width 0.5) (layer F.Cu) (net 14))
 (segment (start 32 45.5) (end 35 48.5) (width 0.5) (layer F.Cu) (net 14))
 (segment (start 32 26) (end 32 45.5) (width 0.5) (layer F.Cu) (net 14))
 (segment (start 29.215 23.215) (end 32 26) (width 0.5) (layer F.Cu) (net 14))
 (segment (start 62.27 26) (end 67 26) (width 0.5) (layer F.Cu) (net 10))
 (segment (start 79.91 18.5) (end 81.41 17) (width 0.5) (layer F.Cu) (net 10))
 (segment (start 74.5 18.5) (end 79.91 18.5) (width 0.5) (layer F.Cu) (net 10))
 (segment (start 67 26) (end 74.5 18.5) (width 0.5) (layer F.Cu) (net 10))
 (segment (start 93.27 49.5) (end 96.65 49.5) (width 0.5) (layer F.Cu) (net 21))
 (segment (start 96.65 49.5) (end 98.15 48) (width 0.5) (layer F.Cu) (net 21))
 (segment (start 119.51 17) (end 119.51 19.8) (width 0.5) (layer B.Cu) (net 3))
 (segment (start 119.51 19.8) (end 115.81 23.5) (width 0.5) (layer B.Cu) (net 3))
 (segment (start 90.81 46) (end 90.81 49.42) (width 0.5) (layer F.Cu) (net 23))
 (segment (start 90.81 49.42) (end 90.73 49.5) (width 0.5) (layer F.Cu) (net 23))
 (segment (start 90.81 46) (end 90.5 46) (width 0.5) (layer F.Cu) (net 23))
 (segment (start 79.51 44) (end 77.51 46) (width 0.5) (layer F.Cu) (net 23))
 (segment (start 88.5 44) (end 79.51 44) (width 0.5) (layer F.Cu) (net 23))
 (segment (start 90.5 46) (end 88.5 44) (width 0.5) (layer F.Cu) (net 23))
 (segment (start 74.97 46) (end 74.97 45.53) (width 0.5) (layer F.Cu) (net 20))
 (segment (start 95.19 42.5) (end 100.69 48) (width 0.5) (layer F.Cu) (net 20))
 (segment (start 78 42.5) (end 95.19 42.5) (width 0.5) (layer F.Cu) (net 20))
 (segment (start 74.97 45.53) (end 78 42.5) (width 0.5) (layer F.Cu) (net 20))
 (segment (start 103.23 48) (end 103 48) (width 0.5) (layer F.Cu) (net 19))
 (segment (start 77.93 40.5) (end 72.43 46) (width 0.5) (layer F.Cu) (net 19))
 (segment (start 95.5 40.5) (end 77.93 40.5) (width 0.5) (layer F.Cu) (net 19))
 (segment (start 103 48) (end 95.5 40.5) (width 0.5) (layer F.Cu) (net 19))
 (segment (start 59.73 26) (end 59.73 25.77) (width 0.5) (layer F.Cu) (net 22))
 (segment (start 66.5 22) (end 66.5 19) (width 0.5) (layer F.Cu) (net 22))
 (segment (start 65 23.5) (end 66.5 22) (width 0.5) (layer F.Cu) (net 22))
 (segment (start 62 23.5) (end 65 23.5) (width 0.5) (layer F.Cu) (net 22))
 (segment (start 59.73 25.77) (end 62 23.5) (width 0.5) (layer F.Cu) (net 22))
 (segment (start 29.805923 36.194077) (end 29.805923 39.194077) (width 0.5) (layer F.Cu) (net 15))
 (segment (start 28.5 40.5) (end 26.785 40.5) (width 0.5) (layer F.Cu) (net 15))
 (segment (start 29.805923 39.194077) (end 28.5 40.5) (width 0.5) (layer F.Cu) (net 15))
 (segment (start 36.285 21.5) (end 36.285 20.215) (width 0.5) (layer F.Cu) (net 11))
 (segment (start 48.69 19) (end 51.19 21.5) (width 0.5) (layer F.Cu) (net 11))
 (segment (start 37.5 19) (end 48.69 19) (width 0.5) (layer F.Cu) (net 11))
 (segment (start 36.285 20.215) (end 37.5 19) (width 0.5) (layer F.Cu) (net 11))
 (segment (start 99.305923 28.694077) (end 97 31) (width 0.5) (layer B.Cu) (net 17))
 (segment (start 91.611846 31) (end 90.305923 32.305923) (width 0.5) (layer B.Cu) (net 17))
 (segment (start 97 31) (end 91.611846 31) (width 0.5) (layer B.Cu) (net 17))
 (segment (start 108.19 23.5) (end 104.888154 23.5) (width 0.5) (layer B.Cu) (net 18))
 (segment (start 104.888154 23.5) (end 104.694077 23.305923) (width 0.5) (layer B.Cu) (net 18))
 (segment (start 24.19 18) (end 21.285 18) (width 0.5) (layer F.Cu) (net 13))
 (segment (start 21.285 18) (end 17.785 21.5) (width 0.5) (layer F.Cu) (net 13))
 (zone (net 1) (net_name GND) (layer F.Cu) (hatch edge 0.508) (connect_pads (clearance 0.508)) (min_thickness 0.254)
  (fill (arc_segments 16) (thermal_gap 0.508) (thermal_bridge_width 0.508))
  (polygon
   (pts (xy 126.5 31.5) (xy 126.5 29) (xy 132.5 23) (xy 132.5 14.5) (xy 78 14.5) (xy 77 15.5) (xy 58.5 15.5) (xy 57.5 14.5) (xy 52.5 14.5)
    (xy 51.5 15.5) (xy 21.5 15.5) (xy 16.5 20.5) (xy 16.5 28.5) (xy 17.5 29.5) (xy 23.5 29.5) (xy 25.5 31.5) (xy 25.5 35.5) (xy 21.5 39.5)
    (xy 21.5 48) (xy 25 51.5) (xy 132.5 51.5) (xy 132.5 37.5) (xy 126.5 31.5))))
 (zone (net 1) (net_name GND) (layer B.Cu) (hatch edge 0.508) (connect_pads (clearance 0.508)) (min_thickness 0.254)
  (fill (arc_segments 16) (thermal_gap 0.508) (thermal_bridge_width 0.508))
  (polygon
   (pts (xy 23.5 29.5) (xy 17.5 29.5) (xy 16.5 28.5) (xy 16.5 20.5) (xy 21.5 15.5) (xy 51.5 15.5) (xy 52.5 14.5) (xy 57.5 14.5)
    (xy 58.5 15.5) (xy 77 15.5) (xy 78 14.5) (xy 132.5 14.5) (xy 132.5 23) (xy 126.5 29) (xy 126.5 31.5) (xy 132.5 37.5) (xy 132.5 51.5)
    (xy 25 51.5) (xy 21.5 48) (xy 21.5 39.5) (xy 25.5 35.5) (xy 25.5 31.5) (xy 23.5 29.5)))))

